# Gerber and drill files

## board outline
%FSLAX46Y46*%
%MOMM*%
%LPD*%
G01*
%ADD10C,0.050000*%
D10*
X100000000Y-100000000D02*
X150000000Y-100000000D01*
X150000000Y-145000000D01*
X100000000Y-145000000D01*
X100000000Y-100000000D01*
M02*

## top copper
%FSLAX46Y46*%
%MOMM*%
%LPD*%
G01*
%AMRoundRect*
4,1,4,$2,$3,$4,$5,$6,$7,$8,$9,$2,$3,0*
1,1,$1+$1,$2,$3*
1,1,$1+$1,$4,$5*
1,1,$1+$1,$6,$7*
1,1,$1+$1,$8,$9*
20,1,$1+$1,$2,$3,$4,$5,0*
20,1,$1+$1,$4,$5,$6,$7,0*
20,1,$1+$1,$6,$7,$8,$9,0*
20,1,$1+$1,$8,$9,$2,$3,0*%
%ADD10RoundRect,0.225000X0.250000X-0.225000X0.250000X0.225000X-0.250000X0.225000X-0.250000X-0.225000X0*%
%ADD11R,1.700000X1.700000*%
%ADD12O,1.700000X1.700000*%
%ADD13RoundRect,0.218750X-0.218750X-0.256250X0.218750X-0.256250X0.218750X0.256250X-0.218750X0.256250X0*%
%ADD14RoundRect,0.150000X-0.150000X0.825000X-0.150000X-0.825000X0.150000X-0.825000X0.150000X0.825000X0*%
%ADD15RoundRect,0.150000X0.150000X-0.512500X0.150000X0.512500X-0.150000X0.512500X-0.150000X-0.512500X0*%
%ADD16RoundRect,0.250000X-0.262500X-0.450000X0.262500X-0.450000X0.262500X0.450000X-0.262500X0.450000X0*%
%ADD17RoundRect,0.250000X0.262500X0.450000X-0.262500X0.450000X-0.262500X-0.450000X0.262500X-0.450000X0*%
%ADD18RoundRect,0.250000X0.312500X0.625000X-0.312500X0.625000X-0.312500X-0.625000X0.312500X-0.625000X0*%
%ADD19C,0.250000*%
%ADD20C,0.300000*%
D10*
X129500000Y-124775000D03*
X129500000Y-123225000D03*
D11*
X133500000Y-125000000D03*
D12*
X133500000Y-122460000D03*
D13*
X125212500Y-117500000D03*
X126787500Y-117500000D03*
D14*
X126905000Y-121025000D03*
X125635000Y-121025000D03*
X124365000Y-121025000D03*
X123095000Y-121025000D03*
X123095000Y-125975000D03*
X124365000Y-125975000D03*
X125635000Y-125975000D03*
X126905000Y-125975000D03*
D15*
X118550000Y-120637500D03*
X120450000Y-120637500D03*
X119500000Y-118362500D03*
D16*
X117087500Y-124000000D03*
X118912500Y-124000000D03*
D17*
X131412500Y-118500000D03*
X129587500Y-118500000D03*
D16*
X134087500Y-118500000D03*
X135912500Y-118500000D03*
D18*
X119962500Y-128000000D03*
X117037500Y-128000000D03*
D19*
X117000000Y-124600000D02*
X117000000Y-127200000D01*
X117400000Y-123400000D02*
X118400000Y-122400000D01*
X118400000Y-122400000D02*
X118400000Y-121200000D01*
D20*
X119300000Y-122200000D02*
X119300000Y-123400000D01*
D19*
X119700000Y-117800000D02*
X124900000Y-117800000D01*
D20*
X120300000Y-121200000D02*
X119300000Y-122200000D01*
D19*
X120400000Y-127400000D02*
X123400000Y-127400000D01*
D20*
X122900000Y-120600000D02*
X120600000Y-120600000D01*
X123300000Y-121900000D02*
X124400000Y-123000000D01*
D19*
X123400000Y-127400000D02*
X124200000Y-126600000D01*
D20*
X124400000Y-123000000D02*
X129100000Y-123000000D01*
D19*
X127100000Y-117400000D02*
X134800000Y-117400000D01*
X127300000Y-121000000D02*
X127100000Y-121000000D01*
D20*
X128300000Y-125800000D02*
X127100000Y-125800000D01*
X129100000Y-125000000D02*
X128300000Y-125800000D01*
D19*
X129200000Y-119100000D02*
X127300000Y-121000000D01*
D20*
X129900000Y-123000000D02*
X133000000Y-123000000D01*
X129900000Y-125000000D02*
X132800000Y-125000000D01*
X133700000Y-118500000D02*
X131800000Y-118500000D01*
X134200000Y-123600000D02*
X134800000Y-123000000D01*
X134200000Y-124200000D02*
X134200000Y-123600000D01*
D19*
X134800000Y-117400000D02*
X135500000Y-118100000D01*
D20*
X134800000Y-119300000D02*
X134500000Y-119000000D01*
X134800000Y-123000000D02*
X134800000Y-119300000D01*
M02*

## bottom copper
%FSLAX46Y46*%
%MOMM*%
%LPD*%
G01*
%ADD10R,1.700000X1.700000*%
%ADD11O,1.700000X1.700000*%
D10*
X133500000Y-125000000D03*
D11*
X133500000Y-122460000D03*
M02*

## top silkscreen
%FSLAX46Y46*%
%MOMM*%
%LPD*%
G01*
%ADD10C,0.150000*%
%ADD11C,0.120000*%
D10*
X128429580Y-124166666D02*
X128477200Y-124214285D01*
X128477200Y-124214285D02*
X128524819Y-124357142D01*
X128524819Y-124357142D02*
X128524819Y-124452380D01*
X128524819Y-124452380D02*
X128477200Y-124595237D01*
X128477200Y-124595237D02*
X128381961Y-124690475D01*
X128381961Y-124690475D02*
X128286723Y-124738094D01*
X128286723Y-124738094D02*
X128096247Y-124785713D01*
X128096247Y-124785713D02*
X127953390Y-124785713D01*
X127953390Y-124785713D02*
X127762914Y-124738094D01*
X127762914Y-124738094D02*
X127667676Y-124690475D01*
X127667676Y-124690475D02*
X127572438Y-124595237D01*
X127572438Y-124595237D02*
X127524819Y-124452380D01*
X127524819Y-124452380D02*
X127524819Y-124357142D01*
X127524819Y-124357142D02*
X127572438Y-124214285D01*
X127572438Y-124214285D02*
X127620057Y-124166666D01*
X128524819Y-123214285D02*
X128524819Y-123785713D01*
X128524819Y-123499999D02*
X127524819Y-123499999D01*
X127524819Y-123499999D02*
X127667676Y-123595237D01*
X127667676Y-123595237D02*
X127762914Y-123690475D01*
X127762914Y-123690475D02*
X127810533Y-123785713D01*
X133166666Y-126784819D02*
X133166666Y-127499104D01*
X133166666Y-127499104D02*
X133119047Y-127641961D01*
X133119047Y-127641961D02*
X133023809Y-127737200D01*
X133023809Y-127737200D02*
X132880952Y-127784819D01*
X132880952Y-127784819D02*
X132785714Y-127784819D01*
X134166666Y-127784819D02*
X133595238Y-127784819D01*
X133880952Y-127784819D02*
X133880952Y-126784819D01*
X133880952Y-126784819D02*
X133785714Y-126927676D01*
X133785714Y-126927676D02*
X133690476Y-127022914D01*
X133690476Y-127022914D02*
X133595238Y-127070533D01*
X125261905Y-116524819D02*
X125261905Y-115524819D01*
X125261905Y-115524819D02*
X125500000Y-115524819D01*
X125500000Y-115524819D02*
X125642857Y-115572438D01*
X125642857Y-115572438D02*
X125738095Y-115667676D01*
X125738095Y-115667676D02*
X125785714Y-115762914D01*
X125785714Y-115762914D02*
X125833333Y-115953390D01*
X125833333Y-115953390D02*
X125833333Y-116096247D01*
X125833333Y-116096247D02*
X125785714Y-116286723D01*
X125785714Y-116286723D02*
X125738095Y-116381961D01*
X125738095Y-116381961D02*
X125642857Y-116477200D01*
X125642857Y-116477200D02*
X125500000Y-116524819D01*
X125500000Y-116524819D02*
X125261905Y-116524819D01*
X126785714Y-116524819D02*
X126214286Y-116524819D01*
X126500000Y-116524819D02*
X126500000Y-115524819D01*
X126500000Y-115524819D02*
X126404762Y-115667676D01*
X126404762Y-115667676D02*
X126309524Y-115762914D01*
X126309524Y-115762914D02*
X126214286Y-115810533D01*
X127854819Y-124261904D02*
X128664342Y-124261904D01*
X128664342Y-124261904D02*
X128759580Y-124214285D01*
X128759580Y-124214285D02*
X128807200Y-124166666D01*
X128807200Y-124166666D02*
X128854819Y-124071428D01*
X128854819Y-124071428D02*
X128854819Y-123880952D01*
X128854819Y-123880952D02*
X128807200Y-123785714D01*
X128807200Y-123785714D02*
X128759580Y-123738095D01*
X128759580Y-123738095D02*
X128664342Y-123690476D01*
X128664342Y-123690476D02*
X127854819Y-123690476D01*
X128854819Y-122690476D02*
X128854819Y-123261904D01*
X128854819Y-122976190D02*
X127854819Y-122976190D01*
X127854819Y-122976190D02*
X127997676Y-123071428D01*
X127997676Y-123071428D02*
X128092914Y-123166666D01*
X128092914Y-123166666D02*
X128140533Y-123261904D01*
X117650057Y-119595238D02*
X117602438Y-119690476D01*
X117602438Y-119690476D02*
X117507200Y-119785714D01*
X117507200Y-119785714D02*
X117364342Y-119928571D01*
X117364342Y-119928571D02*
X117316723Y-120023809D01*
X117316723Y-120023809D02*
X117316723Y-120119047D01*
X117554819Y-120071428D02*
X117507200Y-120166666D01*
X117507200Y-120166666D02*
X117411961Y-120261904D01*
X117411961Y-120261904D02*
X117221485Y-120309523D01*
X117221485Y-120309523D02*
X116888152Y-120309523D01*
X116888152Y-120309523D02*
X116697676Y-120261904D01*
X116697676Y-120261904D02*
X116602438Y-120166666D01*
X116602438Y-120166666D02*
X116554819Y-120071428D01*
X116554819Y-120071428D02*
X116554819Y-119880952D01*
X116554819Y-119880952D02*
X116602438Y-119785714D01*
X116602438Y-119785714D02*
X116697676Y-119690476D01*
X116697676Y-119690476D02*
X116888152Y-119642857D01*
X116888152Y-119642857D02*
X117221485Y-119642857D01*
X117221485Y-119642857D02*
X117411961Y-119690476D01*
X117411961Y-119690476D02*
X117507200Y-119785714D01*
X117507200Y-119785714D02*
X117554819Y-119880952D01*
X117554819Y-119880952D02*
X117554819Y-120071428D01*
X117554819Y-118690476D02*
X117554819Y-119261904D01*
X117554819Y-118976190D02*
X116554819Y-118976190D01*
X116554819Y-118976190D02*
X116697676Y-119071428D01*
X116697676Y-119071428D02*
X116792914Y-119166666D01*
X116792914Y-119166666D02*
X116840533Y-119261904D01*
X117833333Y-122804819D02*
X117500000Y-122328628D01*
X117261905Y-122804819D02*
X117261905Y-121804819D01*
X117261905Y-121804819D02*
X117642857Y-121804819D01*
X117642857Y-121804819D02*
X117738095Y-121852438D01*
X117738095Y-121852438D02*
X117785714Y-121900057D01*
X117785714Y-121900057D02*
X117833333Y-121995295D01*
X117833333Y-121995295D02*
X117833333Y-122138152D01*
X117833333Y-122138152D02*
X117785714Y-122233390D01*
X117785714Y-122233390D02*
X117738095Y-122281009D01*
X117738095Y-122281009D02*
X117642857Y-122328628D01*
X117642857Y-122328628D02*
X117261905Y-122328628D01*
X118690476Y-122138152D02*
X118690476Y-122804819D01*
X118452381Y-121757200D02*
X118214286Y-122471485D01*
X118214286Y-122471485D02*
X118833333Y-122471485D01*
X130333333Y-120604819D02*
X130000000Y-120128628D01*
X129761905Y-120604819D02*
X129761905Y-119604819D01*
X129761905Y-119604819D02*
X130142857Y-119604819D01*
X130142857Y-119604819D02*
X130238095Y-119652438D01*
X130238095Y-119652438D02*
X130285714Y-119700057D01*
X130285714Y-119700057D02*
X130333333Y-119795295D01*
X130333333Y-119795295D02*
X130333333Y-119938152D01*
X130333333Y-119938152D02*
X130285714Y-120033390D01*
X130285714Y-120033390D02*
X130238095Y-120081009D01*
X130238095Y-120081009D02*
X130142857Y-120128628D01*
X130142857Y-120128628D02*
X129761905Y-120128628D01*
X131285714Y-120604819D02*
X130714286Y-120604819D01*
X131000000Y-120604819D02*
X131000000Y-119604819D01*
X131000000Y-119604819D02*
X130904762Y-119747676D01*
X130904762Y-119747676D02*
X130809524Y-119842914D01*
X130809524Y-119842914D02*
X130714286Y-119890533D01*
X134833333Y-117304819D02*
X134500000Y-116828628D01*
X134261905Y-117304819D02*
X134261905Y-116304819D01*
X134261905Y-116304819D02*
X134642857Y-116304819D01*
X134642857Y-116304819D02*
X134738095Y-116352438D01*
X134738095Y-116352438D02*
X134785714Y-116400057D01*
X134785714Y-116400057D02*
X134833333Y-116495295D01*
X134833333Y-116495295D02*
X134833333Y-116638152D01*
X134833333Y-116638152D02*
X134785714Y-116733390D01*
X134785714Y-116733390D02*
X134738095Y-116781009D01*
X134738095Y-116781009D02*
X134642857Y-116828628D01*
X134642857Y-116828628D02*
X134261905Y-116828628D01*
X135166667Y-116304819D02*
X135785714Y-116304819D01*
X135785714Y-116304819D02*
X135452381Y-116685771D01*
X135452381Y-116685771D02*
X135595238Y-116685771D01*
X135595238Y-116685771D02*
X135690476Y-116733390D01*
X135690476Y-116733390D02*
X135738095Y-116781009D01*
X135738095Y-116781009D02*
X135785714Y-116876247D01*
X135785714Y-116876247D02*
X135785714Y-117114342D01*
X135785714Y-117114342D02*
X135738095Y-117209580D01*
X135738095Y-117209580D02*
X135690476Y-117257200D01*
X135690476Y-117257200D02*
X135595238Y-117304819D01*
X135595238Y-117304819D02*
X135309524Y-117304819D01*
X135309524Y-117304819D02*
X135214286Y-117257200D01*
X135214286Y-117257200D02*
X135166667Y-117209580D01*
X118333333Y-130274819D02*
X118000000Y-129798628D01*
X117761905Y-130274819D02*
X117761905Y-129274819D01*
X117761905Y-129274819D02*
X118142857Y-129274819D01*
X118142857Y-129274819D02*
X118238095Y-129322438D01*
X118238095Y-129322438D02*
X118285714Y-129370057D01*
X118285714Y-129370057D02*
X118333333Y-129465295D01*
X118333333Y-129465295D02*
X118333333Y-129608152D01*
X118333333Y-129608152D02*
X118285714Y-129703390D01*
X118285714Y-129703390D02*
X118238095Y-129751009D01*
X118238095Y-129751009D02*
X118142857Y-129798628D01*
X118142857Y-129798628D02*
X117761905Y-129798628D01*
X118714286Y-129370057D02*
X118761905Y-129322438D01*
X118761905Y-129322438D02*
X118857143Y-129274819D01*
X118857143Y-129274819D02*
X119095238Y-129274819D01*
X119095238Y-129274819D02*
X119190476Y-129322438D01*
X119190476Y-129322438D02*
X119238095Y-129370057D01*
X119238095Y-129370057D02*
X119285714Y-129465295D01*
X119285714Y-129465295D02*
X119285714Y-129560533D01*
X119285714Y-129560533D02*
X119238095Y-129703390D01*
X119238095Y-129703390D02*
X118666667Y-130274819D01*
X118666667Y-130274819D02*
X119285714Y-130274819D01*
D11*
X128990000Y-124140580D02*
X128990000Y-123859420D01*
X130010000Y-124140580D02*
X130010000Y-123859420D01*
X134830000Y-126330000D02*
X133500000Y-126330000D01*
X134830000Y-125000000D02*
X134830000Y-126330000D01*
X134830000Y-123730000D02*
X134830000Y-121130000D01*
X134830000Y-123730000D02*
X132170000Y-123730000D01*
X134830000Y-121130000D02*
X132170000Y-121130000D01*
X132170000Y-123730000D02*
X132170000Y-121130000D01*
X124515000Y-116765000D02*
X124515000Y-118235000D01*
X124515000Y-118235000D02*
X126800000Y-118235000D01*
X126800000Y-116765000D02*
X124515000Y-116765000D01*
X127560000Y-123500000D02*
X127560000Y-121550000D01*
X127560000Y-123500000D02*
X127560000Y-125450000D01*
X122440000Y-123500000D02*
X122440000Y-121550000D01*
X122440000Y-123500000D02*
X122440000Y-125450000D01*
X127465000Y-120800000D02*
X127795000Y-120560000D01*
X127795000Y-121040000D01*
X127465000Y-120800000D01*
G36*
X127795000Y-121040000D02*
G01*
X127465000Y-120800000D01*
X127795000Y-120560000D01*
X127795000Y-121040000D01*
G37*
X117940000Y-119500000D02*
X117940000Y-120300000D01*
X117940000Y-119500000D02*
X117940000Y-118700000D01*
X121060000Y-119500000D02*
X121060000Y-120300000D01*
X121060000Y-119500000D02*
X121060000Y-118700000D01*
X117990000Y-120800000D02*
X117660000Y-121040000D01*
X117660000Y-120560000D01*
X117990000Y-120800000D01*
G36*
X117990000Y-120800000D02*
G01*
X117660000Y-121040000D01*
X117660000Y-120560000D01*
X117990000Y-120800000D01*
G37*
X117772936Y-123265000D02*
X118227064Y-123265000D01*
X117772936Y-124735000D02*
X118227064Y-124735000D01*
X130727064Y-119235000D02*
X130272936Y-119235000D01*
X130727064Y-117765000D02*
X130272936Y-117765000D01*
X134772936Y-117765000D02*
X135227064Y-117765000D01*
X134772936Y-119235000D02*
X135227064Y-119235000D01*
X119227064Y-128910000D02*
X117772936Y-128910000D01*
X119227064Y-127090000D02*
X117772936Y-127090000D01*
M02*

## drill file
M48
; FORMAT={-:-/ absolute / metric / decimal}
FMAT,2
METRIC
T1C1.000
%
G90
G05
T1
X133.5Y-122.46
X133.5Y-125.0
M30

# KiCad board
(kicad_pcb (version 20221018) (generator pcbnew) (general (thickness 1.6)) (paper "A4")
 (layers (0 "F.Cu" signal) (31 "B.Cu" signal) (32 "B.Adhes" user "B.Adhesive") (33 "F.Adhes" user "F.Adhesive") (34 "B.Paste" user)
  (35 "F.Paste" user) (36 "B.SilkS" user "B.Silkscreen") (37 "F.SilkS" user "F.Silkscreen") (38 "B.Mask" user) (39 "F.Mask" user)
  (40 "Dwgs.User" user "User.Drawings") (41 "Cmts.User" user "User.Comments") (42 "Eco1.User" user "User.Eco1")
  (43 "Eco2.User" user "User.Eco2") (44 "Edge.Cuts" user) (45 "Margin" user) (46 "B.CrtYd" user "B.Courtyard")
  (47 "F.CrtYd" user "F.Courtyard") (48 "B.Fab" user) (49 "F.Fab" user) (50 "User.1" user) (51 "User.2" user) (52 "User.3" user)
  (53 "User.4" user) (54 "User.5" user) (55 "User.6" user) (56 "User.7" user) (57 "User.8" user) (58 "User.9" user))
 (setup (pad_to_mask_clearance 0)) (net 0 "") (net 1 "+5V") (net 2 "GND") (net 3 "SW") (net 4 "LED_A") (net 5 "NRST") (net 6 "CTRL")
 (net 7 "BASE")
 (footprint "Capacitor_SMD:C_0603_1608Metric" (layer "F.Cu") (at 129.5 124 90)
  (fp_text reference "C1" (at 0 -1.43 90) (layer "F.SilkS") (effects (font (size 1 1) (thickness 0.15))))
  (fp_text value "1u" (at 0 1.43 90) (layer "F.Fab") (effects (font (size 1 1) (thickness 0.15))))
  (fp_line (start -0.14058 -0.51) (end 0.14058 -0.51) (stroke (width 0.12) (type solid)) (layer "F.SilkS"))
  (fp_line (start -0.14058 0.51) (end 0.14058 0.51) (stroke (width 0.12) (type solid)) (layer "F.SilkS"))
  (pad "1" smd roundrect (at -0.775 0 90) (size 0.9 0.95) (layers "F.Cu" "F.Paste" "F.Mask") (roundrect_rratio 0.25) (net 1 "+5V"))
  (pad "2" smd roundrect (at 0.775 0 90) (size 0.9 0.95) (layers "F.Cu" "F.Paste" "F.Mask") (roundrect_rratio 0.25) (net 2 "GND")))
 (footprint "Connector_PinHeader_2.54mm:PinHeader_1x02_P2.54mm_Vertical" (layer "F.Cu") (at 133.5 125 180)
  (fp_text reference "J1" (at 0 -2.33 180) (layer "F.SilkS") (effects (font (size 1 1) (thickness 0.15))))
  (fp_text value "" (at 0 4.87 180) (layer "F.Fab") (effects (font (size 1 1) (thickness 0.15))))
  (fp_line (start -1.33 -1.33) (end 0 -1.33) (stroke (width 0.12) (type solid)) (layer "F.SilkS"))
  (fp_line (start -1.33 0) (end -1.33 -1.33) (stroke (width 0.12) (type solid)) (layer "F.SilkS"))
  (fp_line (start -1.33 1.27) (end -1.33 3.87) (stroke (width 0.12) (type solid)) (layer "F.SilkS"))
  (fp_line (start -1.33 1.27) (end 1.33 1.27) (stroke (width 0.12) (type solid)) (layer "F.SilkS"))
  (fp_line (start -1.33 3.87) (end 1.33 3.87) (stroke (width 0.12) (type solid)) (layer "F.SilkS"))
  (fp_line (start 1.33 1.27) (end 1.33 3.87) (stroke (width 0.12) (type solid)) (layer "F.SilkS"))
  (pad "1" thru_hole rect (at 0 0 180) (size 1.7 1.7) (drill 1) (layers "*.Cu" "*.Mask") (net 1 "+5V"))
  (pad "2" thru_hole oval (at 0 2.54 180) (size 1.7 1.7) (drill 1) (layers "*.Cu" "*.Mask") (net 2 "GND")))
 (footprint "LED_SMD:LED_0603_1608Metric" (layer "F.Cu") (at 126 117.5)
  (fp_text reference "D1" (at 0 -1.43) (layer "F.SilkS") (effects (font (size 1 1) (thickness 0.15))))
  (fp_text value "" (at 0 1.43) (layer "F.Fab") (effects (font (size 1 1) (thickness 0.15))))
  (fp_line (start -1.485 -0.735) (end -1.485 0.735) (stroke (width 0.12) (type solid)) (layer "F.SilkS"))
  (fp_line (start -1.485 0.735) (end 0.8 0.735) (stroke (width 0.12) (type solid)) (layer "F.SilkS"))
  (fp_line (start 0.8 -0.735) (end -1.485 -0.735) (stroke (width 0.12) (type solid)) (layer "F.SilkS"))
  (pad "1" smd roundrect (at -0.7875 0) (size 0.875 0.95) (layers "F.Cu" "F.Paste" "F.Mask") (roundrect_rratio 0.25) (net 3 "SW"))
  (pad "2" smd roundrect (at 0.7875 0) (size 0.875 0.95) (layers "F.Cu" "F.Paste" "F.Mask") (roundrect_rratio 0.25) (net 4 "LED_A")))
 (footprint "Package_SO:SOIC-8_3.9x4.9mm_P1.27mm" (layer "F.Cu") (at 125 123.5 -90)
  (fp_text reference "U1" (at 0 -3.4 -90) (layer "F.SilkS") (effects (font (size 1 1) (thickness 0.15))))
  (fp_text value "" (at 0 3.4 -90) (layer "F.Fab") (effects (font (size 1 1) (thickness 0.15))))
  (fp_line (start 0 -2.56) (end -1.95 -2.56) (stroke (width 0.12) (type solid)) (layer "F.SilkS"))
  (fp_line (start 0 -2.56) (end 1.95 -2.56) (stroke (width 0.12) (type solid)) (layer "F.SilkS"))
  (fp_line (start 0 2.56) (end -1.95 2.56) (stroke (width 0.12) (type solid)) (layer "F.SilkS"))
  (fp_line (start 0 2.56) (end 1.95 2.56) (stroke (width 0.12) (type solid)) (layer "F.SilkS"))
  (fp_poly
   (pts (xy -2.7 -2.465) (xy -2.94 -2.795) (xy -2.46 -2.795) (xy -2.7 -2.465)) (stroke (width 0.12) (type solid)) (fill solid)
   (layer "F.SilkS"))
  (pad "1" smd roundrect (at -2.475 -1.905 270) (size 1.95 0.6) (layers "F.Cu" "F.Paste" "F.Mask") (roundrect_rratio 0.25) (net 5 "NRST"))
  (pad "2" smd roundrect (at -2.475 -0.635 270) (size 1.95 0.6) (layers "F.Cu" "F.Paste" "F.Mask") (roundrect_rratio 0.25))
  (pad "3" smd roundrect (at -2.475 0.635 270) (size 1.95 0.6) (layers "F.Cu" "F.Paste" "F.Mask") (roundrect_rratio 0.25))
  (pad "4" smd roundrect (at -2.475 1.905 270) (size 1.95 0.6) (layers "F.Cu" "F.Paste" "F.Mask") (roundrect_rratio 0.25) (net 2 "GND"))
  (pad "5" smd roundrect (at 2.475 1.905 270) (size 1.95 0.6) (layers "F.Cu" "F.Paste" "F.Mask") (roundrect_rratio 0.25))
  (pad "6" smd roundrect (at 2.475 0.635 270) (size 1.95 0.6) (layers "F.Cu" "F.Paste" "F.Mask") (roundrect_rratio 0.25) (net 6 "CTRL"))
  (pad "7" smd roundrect (at 2.475 -0.635 270) (size 1.95 0.6) (layers "F.Cu" "F.Paste" "F.Mask") (roundrect_rratio 0.25))
  (pad "8" smd roundrect (at 2.475 -1.905 270) (size 1.95 0.6) (layers "F.Cu" "F.Paste" "F.Mask") (roundrect_rratio 0.25) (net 1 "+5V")))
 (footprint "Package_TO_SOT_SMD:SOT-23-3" (layer "F.Cu") (at 119.5 119.5 90)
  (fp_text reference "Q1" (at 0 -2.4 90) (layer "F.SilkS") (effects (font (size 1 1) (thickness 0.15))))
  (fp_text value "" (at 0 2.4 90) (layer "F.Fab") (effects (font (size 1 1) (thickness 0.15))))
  (fp_line (start 0 -1.56) (end -0.8 -1.56) (stroke (width 0.12) (type solid)) (layer "F.SilkS"))
  (fp_line (start 0 -1.56) (end 0.8 -1.56) (stroke (width 0.12) (type solid)) (layer "F.SilkS"))
  (fp_line (start 0 1.56) (end -0.8 1.56) (stroke (width 0.12) (type solid)) (layer "F.SilkS"))
  (fp_line (start 0 1.56) (end 0.8 1.56) (stroke (width 0.12) (type solid)) (layer "F.SilkS"))
  (fp_poly
   (pts (xy -1.3 -1.51) (xy -1.54 -1.84) (xy -1.06 -1.84) (xy -1.3 -1.51)) (stroke (width 0.12) (type solid)) (fill solid) (layer "F.SilkS"))
  (pad "1" smd roundrect (at -1.1375 -0.95 90) (size 1.325 0.6) (layers "F.Cu" "F.Paste" "F.Mask") (roundrect_rratio 0.25) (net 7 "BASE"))
  (pad "2" smd roundrect (at -1.1375 0.95 90) (size 1.325 0.6) (layers "F.Cu" "F.Paste" "F.Mask") (roundrect_rratio 0.25) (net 2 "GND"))
  (pad "3" smd roundrect (at 1.1375 0 90) (size 1.325 0.6) (layers "F.Cu" "F.Paste" "F.Mask") (roundrect_rratio 0.25) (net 3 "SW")))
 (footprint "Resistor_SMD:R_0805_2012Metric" (layer "F.Cu") (at 118 124)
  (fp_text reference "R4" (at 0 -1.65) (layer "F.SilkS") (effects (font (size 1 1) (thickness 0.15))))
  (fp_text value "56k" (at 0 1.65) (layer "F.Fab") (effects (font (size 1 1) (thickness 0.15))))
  (fp_line (start -0.227064 -0.735) (end 0.227064 -0.735) (stroke (width 0.12) (type solid)) (layer "F.SilkS"))
  (fp_line (start -0.227064 0.735) (end 0.227064 0.735) (stroke (width 0.12) (type solid)) (layer "F.SilkS"))
  (pad "1" smd roundrect (at -0.9125 0) (size 1.025 1.4) (layers "F.Cu" "F.Paste" "F.Mask") (roundrect_rratio 0.243902) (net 7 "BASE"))
  (pad "2" smd roundrect (at 0.9125 0) (size 1.025 1.4) (layers "F.Cu" "F.Paste" "F.Mask") (roundrect_rratio 0.243902) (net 2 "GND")))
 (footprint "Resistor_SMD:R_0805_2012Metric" (layer "F.Cu") (at 130.5 118.5 180)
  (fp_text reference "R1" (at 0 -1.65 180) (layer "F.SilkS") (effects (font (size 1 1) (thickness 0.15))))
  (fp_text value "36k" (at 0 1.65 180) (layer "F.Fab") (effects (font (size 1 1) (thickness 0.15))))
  (fp_line (start -0.227064 -0.735) (end 0.227064 -0.735) (stroke (width 0.12) (type solid)) (layer "F.SilkS"))
  (fp_line (start -0.227064 0.735) (end 0.227064 0.735) (stroke (width 0.12) (type solid)) (layer "F.SilkS"))
  (pad "1" smd roundrect (at -0.9125 0 180) (size 1.025 1.4) (layers "F.Cu" "F.Paste" "F.Mask") (roundrect_rratio 0.243902) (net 1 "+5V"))
  (pad "2" smd roundrect (at 0.9125 0 180) (size 1.025 1.4) (layers "F.Cu" "F.Paste" "F.Mask") (roundrect_rratio 0.243902) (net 5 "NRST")))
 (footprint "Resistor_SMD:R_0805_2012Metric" (layer "F.Cu") (at 135 118.5)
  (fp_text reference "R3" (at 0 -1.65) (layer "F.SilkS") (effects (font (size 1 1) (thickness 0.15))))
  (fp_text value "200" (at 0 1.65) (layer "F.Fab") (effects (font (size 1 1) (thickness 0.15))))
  (fp_line (start -0.227064 -0.735) (end 0.227064 -0.735) (stroke (width 0.12) (type solid)) (layer "F.SilkS"))
  (fp_line (start -0.227064 0.735) (end 0.227064 0.735) (stroke (width 0.12) (type solid)) (layer "F.SilkS"))
  (pad "1" smd roundrect (at -0.9125 0) (size 1.025 1.4) (layers "F.Cu" "F.Paste" "F.Mask") (roundrect_rratio 0.243902) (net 1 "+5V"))
  (pad "2" smd roundrect (at 0.9125 0) (size 1.025 1.4) (layers "F.Cu" "F.Paste" "F.Mask") (roundrect_rratio 0.243902) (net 4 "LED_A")))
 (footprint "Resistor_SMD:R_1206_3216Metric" (layer "F.Cu") (at 118.5 128 180)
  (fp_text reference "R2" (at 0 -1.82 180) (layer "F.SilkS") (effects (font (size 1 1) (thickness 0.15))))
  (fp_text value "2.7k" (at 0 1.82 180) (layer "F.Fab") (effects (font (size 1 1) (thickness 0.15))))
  (fp_line (start -0.727064 -0.91) (end 0.727064 -0.91) (stroke (width 0.12) (type solid)) (layer "F.SilkS"))
  (fp_line (start -0.727064 0.91) (end 0.727064 0.91) (stroke (width 0.12) (type solid)) (layer "F.SilkS"))
  (pad "1" smd roundrect (at -1.4625 0 180) (size 1.125 1.75) (layers "F.Cu" "F.Paste" "F.Mask") (roundrect_rratio 0.222222) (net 6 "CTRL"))
  (pad "2" smd roundrect (at 1.4625 0 180) (size 1.125 1.75) (layers "F.Cu" "F.Paste" "F.Mask") (roundrect_rratio 0.222222) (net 7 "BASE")))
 (gr_rect (start 100 100) (end 150 145) (stroke (width 0.05) (type default)) (fill none) (layer "Edge.Cuts"))
 (segment (start 117 124.6) (end 117 127.2) (width 0.25) (layer "F.Cu") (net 7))
 (segment (start 117.4 123.4) (end 118.4 122.4) (width 0.25) (layer "F.Cu") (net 7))
 (segment (start 118.4 122.4) (end 118.4 121.2) (width 0.25) (layer "F.Cu") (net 7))
 (segment (start 119.3 122.2) (end 119.3 123.4) (width 0.3) (layer "F.Cu") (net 2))
 (segment (start 119.7 117.8) (end 124.9 117.8) (width 0.25) (layer "F.Cu") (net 3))
 (segment (start 120.3 121.2) (end 119.3 122.2) (width 0.3) (layer "F.Cu") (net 2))
 (segment (start 120.4 127.4) (end 123.4 127.4) (width 0.25) (layer "F.Cu") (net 6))
 (segment (start 122.9 120.6) (end 120.6 120.6) (width 0.3) (layer "F.Cu") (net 2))
 (segment (start 123.3 121.9) (end 124.4 123) (width 0.3) (layer "F.Cu") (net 2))
 (segment (start 123.4 127.4) (end 124.2 126.6) (width 0.25) (layer "F.Cu") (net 6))
 (segment (start 124.4 123) (end 129.1 123) (width 0.3) (layer "F.Cu") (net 2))
 (segment (start 127.1 117.4) (end 134.8 117.4) (width 0.25) (layer "F.Cu") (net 4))
 (segment (start 127.3 121) (end 127.1 121) (width 0.25) (layer "F.Cu") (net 5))
 (segment (start 128.3 125.8) (end 127.1 125.8) (width 0.3) (layer "F.Cu") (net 1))
 (segment (start 129.1 125) (end 128.3 125.8) (width 0.3) (layer "F.Cu") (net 1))
 (segment (start 129.2 119.1) (end 127.3 121) (width 0.25) (layer "F.Cu") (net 5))
 (segment (start 129.9 123) (end 133 123) (width 0.3) (layer "F.Cu") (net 2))
 (segment (start 129.9 125) (end 132.8 125) (width 0.3) (layer "F.Cu") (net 1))
 (segment (start 133.7 118.5) (end 131.8 118.5) (width 0.3) (layer "F.Cu") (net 1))
 (segment (start 134.2 123.6) (end 134.8 123) (width 0.3) (layer "F.Cu") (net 1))
 (segment (start 134.2 124.2) (end 134.2 123.6) (width 0.3) (layer "F.Cu") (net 1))
 (segment (start 134.8 117.4) (end 135.5 118.1) (width 0.25) (layer "F.Cu") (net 4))
 (segment (start 134.8 119.3) (end 134.5 119) (width 0.3) (layer "F.Cu") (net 1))
 (segment (start 134.8 123) (end 134.8 119.3) (width 0.3) (layer "F.Cu") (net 1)))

